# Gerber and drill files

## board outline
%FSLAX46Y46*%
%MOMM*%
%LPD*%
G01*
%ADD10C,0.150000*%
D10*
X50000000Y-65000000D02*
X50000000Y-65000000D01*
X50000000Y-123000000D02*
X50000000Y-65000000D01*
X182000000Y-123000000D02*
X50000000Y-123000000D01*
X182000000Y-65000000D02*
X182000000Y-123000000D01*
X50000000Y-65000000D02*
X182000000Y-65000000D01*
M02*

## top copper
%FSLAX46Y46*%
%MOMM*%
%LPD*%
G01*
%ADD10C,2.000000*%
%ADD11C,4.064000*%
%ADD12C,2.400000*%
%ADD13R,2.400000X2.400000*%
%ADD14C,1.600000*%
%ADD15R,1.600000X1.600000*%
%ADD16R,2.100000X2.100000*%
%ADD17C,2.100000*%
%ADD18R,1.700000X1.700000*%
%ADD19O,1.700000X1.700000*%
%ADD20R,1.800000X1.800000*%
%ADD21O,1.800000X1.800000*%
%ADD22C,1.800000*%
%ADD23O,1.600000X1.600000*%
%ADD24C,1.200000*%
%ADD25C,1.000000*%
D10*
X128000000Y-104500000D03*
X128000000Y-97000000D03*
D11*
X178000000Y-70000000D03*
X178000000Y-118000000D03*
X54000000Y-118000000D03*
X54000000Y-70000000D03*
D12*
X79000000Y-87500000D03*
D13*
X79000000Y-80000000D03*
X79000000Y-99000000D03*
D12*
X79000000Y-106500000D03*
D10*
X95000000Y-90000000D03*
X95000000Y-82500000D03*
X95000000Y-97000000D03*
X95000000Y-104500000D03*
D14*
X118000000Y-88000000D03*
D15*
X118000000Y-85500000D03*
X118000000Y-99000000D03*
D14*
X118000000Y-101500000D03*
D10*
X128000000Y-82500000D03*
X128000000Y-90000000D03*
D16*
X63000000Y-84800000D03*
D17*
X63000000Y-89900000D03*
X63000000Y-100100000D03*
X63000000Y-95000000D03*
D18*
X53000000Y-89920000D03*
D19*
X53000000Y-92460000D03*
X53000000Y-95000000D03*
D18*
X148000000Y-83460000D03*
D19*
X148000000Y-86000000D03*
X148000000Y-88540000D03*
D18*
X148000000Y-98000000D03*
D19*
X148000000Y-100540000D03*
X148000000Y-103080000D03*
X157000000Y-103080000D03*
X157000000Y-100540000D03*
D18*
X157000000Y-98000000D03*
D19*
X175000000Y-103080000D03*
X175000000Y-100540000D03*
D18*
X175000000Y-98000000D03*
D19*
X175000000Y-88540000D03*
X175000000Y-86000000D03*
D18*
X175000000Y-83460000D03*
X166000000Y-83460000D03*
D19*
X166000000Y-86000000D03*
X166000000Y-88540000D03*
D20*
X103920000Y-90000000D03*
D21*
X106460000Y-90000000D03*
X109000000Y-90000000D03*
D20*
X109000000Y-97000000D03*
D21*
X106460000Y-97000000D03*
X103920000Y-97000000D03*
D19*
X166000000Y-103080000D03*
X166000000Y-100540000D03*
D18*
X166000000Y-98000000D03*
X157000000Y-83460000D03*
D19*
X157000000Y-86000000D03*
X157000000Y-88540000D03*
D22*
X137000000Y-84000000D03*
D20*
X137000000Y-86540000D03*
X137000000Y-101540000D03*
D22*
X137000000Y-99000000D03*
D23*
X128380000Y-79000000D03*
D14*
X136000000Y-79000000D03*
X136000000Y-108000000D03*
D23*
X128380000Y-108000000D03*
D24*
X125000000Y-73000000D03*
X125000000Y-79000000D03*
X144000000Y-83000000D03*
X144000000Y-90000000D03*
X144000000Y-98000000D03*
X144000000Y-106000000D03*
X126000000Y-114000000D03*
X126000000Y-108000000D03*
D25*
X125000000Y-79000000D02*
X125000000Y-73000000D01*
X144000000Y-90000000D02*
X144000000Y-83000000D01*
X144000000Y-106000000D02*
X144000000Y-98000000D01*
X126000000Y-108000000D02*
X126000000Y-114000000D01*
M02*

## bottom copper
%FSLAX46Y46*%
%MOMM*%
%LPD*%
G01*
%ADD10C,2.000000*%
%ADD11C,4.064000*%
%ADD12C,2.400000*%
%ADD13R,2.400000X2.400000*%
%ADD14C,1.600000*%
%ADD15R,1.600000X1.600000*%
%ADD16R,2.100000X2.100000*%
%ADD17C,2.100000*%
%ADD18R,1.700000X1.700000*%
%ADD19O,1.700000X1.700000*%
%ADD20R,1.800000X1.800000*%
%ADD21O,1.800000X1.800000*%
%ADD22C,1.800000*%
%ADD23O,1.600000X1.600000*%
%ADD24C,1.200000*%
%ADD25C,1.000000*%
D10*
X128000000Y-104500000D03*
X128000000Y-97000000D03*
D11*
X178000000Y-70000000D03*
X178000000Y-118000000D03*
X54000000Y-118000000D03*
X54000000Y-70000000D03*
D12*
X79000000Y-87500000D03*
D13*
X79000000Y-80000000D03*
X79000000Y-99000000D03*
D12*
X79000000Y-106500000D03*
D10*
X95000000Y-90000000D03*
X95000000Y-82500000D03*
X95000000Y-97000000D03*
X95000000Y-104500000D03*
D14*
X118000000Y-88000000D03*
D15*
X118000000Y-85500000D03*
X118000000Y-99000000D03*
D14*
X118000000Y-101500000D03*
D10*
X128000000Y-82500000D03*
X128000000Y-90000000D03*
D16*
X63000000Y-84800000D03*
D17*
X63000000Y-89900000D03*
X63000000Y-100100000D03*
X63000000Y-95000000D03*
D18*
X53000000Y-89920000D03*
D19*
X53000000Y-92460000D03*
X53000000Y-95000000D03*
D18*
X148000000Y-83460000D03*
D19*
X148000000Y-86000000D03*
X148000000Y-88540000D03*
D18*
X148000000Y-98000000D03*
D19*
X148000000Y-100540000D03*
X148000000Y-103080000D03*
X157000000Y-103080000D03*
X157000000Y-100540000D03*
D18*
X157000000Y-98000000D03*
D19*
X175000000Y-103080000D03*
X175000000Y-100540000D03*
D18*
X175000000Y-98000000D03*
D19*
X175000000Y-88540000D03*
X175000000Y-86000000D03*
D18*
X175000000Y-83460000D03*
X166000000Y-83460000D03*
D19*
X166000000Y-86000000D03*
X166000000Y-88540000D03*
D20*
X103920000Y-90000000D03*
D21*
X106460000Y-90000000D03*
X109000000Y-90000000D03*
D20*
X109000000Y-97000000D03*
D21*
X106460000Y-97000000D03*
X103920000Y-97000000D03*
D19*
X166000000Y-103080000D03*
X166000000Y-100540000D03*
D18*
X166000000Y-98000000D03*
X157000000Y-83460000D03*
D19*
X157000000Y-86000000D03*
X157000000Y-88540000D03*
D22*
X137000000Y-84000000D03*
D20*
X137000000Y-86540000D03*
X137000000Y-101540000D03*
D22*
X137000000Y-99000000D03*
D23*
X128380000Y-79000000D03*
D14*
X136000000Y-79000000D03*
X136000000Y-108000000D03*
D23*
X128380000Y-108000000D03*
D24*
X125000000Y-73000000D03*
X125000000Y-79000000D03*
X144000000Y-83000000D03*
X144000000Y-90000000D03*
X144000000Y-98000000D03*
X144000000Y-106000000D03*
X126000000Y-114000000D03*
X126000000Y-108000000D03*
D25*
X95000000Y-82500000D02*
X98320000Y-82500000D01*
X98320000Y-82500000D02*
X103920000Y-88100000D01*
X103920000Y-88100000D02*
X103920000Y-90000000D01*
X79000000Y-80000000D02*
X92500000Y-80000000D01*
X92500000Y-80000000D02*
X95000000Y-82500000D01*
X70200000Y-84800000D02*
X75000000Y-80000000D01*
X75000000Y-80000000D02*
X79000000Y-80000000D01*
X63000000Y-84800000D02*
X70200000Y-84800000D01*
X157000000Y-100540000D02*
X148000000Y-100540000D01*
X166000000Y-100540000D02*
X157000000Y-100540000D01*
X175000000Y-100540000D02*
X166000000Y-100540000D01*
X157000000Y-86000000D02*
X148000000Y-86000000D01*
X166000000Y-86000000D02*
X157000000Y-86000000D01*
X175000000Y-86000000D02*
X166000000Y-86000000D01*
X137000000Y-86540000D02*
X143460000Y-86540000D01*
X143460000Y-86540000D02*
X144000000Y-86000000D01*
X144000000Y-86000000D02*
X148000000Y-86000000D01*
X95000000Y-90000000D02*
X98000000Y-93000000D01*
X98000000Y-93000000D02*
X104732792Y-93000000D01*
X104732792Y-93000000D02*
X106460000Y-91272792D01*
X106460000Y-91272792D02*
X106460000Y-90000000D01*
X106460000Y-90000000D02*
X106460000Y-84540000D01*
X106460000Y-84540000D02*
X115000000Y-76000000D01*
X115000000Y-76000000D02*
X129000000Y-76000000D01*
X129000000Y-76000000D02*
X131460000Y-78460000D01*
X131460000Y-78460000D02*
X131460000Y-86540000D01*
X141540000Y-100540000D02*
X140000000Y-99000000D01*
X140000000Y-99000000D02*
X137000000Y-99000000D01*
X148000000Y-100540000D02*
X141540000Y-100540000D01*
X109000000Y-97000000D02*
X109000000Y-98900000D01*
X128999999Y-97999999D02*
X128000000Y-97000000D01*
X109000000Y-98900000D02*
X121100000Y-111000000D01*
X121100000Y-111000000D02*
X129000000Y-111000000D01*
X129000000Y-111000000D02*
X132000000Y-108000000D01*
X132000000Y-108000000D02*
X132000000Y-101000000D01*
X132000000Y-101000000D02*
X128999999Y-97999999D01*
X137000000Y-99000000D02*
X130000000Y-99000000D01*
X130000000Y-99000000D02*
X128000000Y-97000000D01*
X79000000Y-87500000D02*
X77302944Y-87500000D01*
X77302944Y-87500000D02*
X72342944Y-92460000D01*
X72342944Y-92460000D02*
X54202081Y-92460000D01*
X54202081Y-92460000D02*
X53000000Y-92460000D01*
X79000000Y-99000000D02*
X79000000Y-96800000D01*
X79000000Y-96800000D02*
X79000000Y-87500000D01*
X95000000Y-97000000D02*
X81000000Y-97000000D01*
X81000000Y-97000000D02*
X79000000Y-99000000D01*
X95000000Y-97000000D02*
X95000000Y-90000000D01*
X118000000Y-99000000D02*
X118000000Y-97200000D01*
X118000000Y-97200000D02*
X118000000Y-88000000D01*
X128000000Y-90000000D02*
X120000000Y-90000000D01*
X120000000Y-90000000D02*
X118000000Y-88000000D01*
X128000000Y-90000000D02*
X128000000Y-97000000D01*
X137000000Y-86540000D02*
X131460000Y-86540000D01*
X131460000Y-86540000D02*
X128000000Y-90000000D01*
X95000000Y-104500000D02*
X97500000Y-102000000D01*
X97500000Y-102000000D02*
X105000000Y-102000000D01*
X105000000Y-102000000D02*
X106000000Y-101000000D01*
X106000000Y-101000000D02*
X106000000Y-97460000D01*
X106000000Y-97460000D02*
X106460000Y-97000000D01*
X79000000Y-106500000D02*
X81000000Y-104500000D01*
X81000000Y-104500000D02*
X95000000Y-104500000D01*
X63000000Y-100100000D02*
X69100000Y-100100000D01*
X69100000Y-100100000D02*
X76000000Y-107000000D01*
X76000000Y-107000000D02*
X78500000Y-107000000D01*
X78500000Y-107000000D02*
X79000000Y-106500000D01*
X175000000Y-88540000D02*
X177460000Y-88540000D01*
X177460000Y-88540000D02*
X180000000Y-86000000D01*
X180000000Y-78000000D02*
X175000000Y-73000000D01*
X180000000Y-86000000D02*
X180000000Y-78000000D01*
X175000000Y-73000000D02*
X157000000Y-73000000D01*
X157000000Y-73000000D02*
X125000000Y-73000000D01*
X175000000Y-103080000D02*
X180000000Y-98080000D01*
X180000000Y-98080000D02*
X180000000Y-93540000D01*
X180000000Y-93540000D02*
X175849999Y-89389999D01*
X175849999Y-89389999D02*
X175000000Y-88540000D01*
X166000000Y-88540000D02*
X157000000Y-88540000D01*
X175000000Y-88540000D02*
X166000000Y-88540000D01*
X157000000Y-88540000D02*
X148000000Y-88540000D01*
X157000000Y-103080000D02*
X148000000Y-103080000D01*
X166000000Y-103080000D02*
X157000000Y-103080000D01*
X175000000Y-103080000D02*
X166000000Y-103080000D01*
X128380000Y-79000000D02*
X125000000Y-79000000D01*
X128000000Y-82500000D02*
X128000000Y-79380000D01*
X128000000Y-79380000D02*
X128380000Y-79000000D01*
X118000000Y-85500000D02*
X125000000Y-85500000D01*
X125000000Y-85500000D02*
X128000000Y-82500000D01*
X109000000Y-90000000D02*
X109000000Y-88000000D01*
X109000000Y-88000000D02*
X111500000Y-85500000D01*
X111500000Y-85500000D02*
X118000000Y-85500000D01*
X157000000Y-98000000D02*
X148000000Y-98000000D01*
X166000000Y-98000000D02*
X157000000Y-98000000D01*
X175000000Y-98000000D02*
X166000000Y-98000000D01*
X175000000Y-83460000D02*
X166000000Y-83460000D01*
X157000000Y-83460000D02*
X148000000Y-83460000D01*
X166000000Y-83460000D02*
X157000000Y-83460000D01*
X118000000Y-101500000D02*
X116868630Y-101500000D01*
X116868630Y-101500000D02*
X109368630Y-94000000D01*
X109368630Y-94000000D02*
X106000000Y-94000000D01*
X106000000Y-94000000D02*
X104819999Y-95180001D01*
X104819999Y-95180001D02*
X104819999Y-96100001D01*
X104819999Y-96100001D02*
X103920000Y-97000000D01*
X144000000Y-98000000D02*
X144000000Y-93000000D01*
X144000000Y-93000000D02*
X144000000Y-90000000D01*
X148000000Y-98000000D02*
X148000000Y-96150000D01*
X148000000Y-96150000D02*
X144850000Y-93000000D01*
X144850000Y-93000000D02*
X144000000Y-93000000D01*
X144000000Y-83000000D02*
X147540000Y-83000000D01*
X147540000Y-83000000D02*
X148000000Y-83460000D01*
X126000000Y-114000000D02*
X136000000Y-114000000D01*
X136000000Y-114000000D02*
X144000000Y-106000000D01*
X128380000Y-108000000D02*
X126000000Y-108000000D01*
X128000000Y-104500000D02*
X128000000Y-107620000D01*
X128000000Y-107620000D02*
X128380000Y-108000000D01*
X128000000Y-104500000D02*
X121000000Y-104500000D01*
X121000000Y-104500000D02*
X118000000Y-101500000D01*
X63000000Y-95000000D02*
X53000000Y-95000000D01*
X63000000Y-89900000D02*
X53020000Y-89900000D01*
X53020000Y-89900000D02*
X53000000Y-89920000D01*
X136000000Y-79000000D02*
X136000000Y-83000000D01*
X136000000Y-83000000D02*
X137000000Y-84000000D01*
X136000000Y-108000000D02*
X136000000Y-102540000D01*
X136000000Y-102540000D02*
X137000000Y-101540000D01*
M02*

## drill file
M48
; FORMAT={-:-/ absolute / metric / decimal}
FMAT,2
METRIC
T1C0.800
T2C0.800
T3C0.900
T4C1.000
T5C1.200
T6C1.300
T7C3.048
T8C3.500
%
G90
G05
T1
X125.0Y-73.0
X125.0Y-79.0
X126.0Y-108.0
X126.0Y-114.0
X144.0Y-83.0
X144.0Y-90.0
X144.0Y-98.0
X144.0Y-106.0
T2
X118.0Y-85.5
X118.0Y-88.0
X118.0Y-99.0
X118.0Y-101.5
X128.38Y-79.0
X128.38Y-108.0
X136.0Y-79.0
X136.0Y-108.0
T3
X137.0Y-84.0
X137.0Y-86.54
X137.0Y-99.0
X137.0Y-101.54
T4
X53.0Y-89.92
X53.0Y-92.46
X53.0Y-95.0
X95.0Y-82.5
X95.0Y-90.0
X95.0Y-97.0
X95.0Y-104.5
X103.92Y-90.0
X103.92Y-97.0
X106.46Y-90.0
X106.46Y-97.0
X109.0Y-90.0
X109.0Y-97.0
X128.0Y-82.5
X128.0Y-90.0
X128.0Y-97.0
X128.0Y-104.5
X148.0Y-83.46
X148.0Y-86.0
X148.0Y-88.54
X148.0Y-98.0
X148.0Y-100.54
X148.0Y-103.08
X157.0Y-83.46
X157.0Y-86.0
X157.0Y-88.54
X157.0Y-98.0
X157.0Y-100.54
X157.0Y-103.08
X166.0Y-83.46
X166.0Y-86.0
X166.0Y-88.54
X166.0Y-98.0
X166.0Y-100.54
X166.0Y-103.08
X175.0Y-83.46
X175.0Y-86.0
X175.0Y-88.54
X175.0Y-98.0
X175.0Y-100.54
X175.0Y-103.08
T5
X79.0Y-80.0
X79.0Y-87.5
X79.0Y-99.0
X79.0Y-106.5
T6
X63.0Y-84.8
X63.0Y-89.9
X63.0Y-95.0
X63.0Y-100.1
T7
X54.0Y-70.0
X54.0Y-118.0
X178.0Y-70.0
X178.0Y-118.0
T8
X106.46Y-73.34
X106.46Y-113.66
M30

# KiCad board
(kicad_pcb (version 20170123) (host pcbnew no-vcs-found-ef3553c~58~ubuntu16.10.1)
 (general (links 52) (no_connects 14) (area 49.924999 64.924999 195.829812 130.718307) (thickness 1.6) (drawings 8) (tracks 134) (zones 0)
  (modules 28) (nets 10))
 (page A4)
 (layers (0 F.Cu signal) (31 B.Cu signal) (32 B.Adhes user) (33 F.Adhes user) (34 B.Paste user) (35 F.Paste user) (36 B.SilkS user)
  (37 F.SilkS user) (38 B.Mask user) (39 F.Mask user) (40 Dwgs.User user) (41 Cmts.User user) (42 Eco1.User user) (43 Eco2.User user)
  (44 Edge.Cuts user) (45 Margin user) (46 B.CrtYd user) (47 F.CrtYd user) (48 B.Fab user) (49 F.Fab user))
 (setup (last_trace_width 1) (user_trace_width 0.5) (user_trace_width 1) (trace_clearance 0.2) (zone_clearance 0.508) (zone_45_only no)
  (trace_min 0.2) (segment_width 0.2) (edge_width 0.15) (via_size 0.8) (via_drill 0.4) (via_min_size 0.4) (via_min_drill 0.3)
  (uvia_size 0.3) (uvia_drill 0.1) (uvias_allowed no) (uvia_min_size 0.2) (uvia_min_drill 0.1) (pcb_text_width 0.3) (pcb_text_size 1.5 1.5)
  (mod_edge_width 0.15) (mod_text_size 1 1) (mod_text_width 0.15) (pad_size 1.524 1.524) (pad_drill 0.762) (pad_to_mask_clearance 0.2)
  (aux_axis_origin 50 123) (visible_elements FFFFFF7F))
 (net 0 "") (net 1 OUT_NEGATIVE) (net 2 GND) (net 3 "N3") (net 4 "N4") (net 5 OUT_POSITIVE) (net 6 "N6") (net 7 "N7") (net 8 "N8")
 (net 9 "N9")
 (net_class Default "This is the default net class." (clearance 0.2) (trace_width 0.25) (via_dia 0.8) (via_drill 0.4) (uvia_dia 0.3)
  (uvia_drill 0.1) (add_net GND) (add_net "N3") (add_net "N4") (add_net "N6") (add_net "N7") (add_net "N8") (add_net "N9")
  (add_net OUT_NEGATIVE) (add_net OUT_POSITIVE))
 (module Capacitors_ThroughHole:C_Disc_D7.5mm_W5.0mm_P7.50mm (layer F.Cu) (at 128 97 270)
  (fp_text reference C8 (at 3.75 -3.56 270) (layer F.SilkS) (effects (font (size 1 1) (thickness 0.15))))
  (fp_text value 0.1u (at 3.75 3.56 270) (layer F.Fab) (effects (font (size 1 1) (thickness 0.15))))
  (pad 2 thru_hole circle (at 7.5 0 270) (size 2 2) (drill 1) (layers *.Cu *.Mask) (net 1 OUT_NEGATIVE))
  (pad 1 thru_hole circle (at 0 0 270) (size 2 2) (drill 1) (layers *.Cu *.Mask) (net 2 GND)))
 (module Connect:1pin (layer F.Cu) (at 178 70)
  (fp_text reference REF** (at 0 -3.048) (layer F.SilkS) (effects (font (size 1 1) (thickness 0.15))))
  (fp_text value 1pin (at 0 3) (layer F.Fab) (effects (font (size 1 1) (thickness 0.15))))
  (pad 1 thru_hole circle (at 0 0) (size 4.064 4.064) (drill 3.048) (layers *.Cu *.Mask)))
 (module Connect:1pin (layer F.Cu) (at 178 118)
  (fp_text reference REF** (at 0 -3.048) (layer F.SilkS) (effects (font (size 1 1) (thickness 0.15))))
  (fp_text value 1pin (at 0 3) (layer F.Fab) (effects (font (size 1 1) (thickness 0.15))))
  (pad 1 thru_hole circle (at 0 0) (size 4.064 4.064) (drill 3.048) (layers *.Cu *.Mask)))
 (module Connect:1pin (layer F.Cu) (at 54 118)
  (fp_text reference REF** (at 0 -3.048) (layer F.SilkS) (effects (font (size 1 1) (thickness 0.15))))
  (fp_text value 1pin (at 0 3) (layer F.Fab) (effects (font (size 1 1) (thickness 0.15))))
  (pad 1 thru_hole circle (at 0 0) (size 4.064 4.064) (drill 3.048) (layers *.Cu *.Mask)))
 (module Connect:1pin (layer F.Cu) (at 54 70)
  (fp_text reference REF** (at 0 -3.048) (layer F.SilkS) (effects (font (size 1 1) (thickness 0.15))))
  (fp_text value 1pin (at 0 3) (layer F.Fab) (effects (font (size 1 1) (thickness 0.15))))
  (pad 1 thru_hole circle (at 0 0) (size 4.064 4.064) (drill 3.048) (layers *.Cu *.Mask)))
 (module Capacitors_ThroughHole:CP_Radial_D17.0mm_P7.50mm (layer F.Cu) (at 79 80 270)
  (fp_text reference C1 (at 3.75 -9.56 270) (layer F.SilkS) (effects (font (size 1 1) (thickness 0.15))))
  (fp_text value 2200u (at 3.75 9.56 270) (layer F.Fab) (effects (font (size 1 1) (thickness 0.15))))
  (pad 2 thru_hole circle (at 7.5 0 270) (size 2.4 2.4) (drill 1.2) (layers *.Cu *.Mask) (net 2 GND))
  (pad 1 thru_hole rect (at 0 0 270) (size 2.4 2.4) (drill 1.2) (layers *.Cu *.Mask) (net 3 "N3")))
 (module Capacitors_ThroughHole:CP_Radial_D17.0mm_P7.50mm (layer F.Cu) (at 79 99 270)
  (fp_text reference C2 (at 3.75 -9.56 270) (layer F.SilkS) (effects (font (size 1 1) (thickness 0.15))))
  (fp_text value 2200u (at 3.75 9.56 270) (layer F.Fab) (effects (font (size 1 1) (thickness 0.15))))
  (pad 1 thru_hole rect (at 0 0 270) (size 2.4 2.4) (drill 1.2) (layers *.Cu *.Mask) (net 2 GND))
  (pad 2 thru_hole circle (at 7.5 0 270) (size 2.4 2.4) (drill 1.2) (layers *.Cu *.Mask) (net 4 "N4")))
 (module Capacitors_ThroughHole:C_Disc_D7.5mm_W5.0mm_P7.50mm (layer F.Cu) (at 95 82.5 270)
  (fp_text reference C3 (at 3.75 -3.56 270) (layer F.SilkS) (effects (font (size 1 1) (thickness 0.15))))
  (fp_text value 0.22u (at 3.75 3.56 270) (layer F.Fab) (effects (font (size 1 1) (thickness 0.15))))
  (pad 2 thru_hole circle (at 7.5 0 270) (size 2 2) (drill 1) (layers *.Cu *.Mask) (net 2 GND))
  (pad 1 thru_hole circle (at 0 0 270) (size 2 2) (drill 1) (layers *.Cu *.Mask) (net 3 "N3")))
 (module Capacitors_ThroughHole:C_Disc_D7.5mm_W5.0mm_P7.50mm (layer F.Cu) (at 95 97 270)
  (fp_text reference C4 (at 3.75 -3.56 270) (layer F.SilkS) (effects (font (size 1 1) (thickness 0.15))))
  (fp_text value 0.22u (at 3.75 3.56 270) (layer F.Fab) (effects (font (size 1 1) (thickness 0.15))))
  (pad 1 thru_hole circle (at 0 0 270) (size 2 2) (drill 1) (layers *.Cu *.Mask) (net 2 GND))
  (pad 2 thru_hole circle (at 7.5 0 270) (size 2 2) (drill 1) (layers *.Cu *.Mask) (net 4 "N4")))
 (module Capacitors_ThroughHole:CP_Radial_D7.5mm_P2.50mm (layer F.Cu) (at 118 85.5 270)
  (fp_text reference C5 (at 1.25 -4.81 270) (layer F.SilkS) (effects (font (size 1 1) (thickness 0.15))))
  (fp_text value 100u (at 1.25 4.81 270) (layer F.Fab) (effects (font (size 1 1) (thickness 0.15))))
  (pad 2 thru_hole circle (at 2.5 0 270) (size 1.6 1.6) (drill 0.8) (layers *.Cu *.Mask) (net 2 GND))
  (pad 1 thru_hole rect (at 0 0 270) (size 1.6 1.6) (drill 0.8) (layers *.Cu *.Mask) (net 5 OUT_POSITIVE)))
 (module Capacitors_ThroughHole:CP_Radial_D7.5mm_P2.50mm (layer F.Cu) (at 118 99 270)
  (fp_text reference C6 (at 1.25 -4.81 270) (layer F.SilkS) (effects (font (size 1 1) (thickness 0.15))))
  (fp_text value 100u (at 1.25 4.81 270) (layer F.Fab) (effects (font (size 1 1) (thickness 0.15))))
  (pad 1 thru_hole rect (at 0 0 270) (size 1.6 1.6) (drill 0.8) (layers *.Cu *.Mask) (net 2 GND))
  (pad 2 thru_hole circle (at 2.5 0 270) (size 1.6 1.6) (drill 0.8) (layers *.Cu *.Mask) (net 1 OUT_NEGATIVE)))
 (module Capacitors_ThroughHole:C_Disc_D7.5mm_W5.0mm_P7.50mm (layer F.Cu) (at 128 82.5 270)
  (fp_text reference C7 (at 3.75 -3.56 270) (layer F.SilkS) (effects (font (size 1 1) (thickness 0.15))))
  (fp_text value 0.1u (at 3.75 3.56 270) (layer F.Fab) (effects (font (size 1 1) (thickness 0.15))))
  (pad 1 thru_hole circle (at 0 0 270) (size 2 2) (drill 1) (layers *.Cu *.Mask) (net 5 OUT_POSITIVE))
  (pad 2 thru_hole circle (at 7.5 0 270) (size 2 2) (drill 1) (layers *.Cu *.Mask) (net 2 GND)))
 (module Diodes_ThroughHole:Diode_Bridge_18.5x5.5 (layer F.Cu) (at 63 84.8 270)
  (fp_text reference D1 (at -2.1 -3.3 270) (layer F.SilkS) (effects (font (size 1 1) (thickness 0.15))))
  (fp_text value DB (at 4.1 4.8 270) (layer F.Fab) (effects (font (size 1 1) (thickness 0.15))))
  (pad 3 thru_hole rect (at 0 0 270) (size 2.1 2.1) (drill 1.3) (layers *.Cu *.Mask) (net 3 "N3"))
  (pad 2 thru_hole circle (at 5.1 0 270) (size 2.1 2.1) (drill 1.3) (layers *.Cu *.Mask) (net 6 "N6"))
  (pad 1 thru_hole circle (at 15.3 0 270) (size 2.1 2.1) (drill 1.3) (layers *.Cu *.Mask) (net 4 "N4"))
  (pad 4 thru_hole circle (at 10.2 0 270) (size 2.1 2.1) (drill 1.3) (layers *.Cu *.Mask) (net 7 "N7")))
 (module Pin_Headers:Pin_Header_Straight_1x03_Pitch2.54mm (layer F.Cu) (at 53 89.92)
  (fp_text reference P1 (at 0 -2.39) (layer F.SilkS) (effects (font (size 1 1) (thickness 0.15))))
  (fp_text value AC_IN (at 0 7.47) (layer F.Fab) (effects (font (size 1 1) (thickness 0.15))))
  (pad 1 thru_hole rect (at 0 0) (size 1.7 1.7) (drill 1) (layers *.Cu *.Mask) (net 6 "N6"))
  (pad 2 thru_hole oval (at 0 2.54) (size 1.7 1.7) (drill 1) (layers *.Cu *.Mask) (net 2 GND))
  (pad 3 thru_hole oval (at 0 5.08) (size 1.7 1.7) (drill 1) (layers *.Cu *.Mask) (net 7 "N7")))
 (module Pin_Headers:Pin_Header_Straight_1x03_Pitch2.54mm (layer F.Cu) (at 148 83.46)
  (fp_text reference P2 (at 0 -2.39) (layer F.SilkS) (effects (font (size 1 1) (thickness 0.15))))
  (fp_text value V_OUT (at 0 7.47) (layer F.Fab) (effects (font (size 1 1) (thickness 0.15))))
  (pad 1 thru_hole rect (at 0 0) (size 1.7 1.7) (drill 1) (layers *.Cu *.Mask) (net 1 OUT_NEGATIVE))
  (pad 2 thru_hole oval (at 0 2.54) (size 1.7 1.7) (drill 1) (layers *.Cu *.Mask) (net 2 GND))
  (pad 3 thru_hole oval (at 0 5.08) (size 1.7 1.7) (drill 1) (layers *.Cu *.Mask) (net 5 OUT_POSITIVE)))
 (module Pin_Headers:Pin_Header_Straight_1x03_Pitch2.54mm (layer F.Cu) (at 148 98)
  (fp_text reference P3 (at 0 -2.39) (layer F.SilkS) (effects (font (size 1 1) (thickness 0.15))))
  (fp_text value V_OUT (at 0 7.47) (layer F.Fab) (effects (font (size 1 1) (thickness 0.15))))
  (pad 1 thru_hole rect (at 0 0) (size 1.7 1.7) (drill 1) (layers *.Cu *.Mask) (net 1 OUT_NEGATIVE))
  (pad 2 thru_hole oval (at 0 2.54) (size 1.7 1.7) (drill 1) (layers *.Cu *.Mask) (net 2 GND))
  (pad 3 thru_hole oval (at 0 5.08) (size 1.7 1.7) (drill 1) (layers *.Cu *.Mask) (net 5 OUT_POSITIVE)))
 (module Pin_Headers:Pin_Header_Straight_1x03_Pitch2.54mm (layer F.Cu) (at 157 98)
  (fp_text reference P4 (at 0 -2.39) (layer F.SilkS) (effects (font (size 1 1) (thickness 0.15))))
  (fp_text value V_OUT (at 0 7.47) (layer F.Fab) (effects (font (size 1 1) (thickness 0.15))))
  (pad 3 thru_hole oval (at 0 5.08) (size 1.7 1.7) (drill 1) (layers *.Cu *.Mask) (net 5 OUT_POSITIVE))
  (pad 2 thru_hole oval (at 0 2.54) (size 1.7 1.7) (drill 1) (layers *.Cu *.Mask) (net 2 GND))
  (pad 1 thru_hole rect (at 0 0) (size 1.7 1.7) (drill 1) (layers *.Cu *.Mask) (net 1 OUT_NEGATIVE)))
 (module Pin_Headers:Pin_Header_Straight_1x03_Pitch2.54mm (layer F.Cu) (at 175 98)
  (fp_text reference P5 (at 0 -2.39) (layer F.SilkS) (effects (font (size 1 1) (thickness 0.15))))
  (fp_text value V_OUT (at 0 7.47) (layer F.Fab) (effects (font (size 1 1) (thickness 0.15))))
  (pad 3 thru_hole oval (at 0 5.08) (size 1.7 1.7) (drill 1) (layers *.Cu *.Mask) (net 5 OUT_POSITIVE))
  (pad 2 thru_hole oval (at 0 2.54) (size 1.7 1.7) (drill 1) (layers *.Cu *.Mask) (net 2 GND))
  (pad 1 thru_hole rect (at 0 0) (size 1.7 1.7) (drill 1) (layers *.Cu *.Mask) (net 1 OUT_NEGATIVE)))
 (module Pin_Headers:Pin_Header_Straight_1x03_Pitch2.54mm (layer F.Cu) (at 175 83.46)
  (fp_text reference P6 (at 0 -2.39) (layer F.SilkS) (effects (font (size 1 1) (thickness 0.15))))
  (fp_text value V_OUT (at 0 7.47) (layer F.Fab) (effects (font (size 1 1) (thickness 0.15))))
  (pad 3 thru_hole oval (at 0 5.08) (size 1.7 1.7) (drill 1) (layers *.Cu *.Mask) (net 5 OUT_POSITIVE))
  (pad 2 thru_hole oval (at 0 2.54) (size 1.7 1.7) (drill 1) (layers *.Cu *.Mask) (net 2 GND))
  (pad 1 thru_hole rect (at 0 0) (size 1.7 1.7) (drill 1) (layers *.Cu *.Mask) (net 1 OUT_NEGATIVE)))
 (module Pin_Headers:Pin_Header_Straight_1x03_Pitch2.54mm (layer F.Cu) (at 166 83.46)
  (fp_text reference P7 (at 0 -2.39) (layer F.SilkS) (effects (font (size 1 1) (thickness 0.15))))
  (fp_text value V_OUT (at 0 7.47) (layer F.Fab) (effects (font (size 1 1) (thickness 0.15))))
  (pad 1 thru_hole rect (at 0 0) (size 1.7 1.7) (drill 1) (layers *.Cu *.Mask) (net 1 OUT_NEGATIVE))
  (pad 2 thru_hole oval (at 0 2.54) (size 1.7 1.7) (drill 1) (layers *.Cu *.Mask) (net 2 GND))
  (pad 3 thru_hole oval (at 0 5.08) (size 1.7 1.7) (drill 1) (layers *.Cu *.Mask) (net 5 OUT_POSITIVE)))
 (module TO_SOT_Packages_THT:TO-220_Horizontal (layer F.Cu) (at 103.92 90)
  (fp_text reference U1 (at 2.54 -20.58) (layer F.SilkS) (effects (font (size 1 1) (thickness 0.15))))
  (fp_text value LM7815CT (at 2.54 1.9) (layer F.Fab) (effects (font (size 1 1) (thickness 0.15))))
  (pad None np_thru_hole oval (at 2.54 -16.66) (size 3.5 3.5) (drill 3.5) (layers *.Cu *.Mask))
  (pad 1 thru_hole rect (at 0 0) (size 1.8 1.8) (drill 1) (layers *.Cu *.Mask) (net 3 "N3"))
  (pad 2 thru_hole oval (at 2.54 0) (size 1.8 1.8) (drill 1) (layers *.Cu *.Mask) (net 2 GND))
  (pad 3 thru_hole oval (at 5.08 0) (size 1.8 1.8) (drill 1) (layers *.Cu *.Mask) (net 5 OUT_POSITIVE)))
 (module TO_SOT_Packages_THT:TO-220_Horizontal (layer F.Cu) (at 109 97 180)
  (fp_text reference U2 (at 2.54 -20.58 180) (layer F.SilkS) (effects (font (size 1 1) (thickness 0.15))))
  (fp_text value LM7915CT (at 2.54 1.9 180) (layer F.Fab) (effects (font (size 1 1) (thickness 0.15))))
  (pad None np_thru_hole oval (at 2.54 -16.66 180) (size 3.5 3.5) (drill 3.5) (layers *.Cu *.Mask))
  (pad 1 thru_hole rect (at 0 0 180) (size 1.8 1.8) (drill 1) (layers *.Cu *.Mask) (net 2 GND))
  (pad 2 thru_hole oval (at 2.54 0 180) (size 1.8 1.8) (drill 1) (layers *.Cu *.Mask) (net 4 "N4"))
  (pad 3 thru_hole oval (at 5.08 0 180) (size 1.8 1.8) (drill 1) (layers *.Cu *.Mask) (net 1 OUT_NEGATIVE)))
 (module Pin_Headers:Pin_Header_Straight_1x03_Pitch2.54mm (layer F.Cu) (at 166 98)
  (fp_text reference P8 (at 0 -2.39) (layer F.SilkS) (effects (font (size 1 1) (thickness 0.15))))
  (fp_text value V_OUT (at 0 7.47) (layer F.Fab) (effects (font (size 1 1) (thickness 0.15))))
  (pad 3 thru_hole oval (at 0 5.08) (size 1.7 1.7) (drill 1) (layers *.Cu *.Mask) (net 5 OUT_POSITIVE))
  (pad 2 thru_hole oval (at 0 2.54) (size 1.7 1.7) (drill 1) (layers *.Cu *.Mask) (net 2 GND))
  (pad 1 thru_hole rect (at 0 0) (size 1.7 1.7) (drill 1) (layers *.Cu *.Mask) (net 1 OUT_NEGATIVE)))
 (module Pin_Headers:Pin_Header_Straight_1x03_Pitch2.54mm (layer F.Cu) (at 157 83.46)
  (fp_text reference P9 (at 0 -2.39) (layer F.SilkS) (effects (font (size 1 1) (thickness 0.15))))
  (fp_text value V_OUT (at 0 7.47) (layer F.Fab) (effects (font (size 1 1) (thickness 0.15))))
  (pad 1 thru_hole rect (at 0 0) (size 1.7 1.7) (drill 1) (layers *.Cu *.Mask) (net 1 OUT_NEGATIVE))
  (pad 2 thru_hole oval (at 0 2.54) (size 1.7 1.7) (drill 1) (layers *.Cu *.Mask) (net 2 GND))
  (pad 3 thru_hole oval (at 0 5.08) (size 1.7 1.7) (drill 1) (layers *.Cu *.Mask) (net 5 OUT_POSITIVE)))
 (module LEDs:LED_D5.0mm (layer F.Cu) (at 137 86.54 90)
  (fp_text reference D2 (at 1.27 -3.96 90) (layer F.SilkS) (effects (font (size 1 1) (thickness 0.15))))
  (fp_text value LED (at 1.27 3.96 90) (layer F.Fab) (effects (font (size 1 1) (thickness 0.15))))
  (pad 2 thru_hole circle (at 2.54 0 90) (size 1.8 1.8) (drill 0.9) (layers *.Cu *.Mask) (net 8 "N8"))
  (pad 1 thru_hole rect (at 0 0 90) (size 1.8 1.8) (drill 0.9) (layers *.Cu *.Mask) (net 2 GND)))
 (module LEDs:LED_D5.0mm (layer F.Cu) (at 137 101.54 90)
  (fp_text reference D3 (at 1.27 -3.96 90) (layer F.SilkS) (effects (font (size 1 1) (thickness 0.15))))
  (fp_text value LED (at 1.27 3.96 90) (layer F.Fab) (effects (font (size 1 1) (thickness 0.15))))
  (pad 1 thru_hole rect (at 0 0 90) (size 1.8 1.8) (drill 0.9) (layers *.Cu *.Mask) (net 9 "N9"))
  (pad 2 thru_hole circle (at 2.54 0 90) (size 1.8 1.8) (drill 0.9) (layers *.Cu *.Mask) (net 2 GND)))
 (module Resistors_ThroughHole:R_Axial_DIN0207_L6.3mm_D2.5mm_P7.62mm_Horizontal (layer F.Cu) (at 136 79 180)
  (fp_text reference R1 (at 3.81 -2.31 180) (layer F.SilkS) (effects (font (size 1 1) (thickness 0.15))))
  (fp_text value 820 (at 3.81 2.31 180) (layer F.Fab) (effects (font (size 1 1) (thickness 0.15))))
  (pad 2 thru_hole oval (at 7.62 0 180) (size 1.6 1.6) (drill 0.8) (layers *.Cu *.Mask) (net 5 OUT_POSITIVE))
  (pad 1 thru_hole circle (at 0 0 180) (size 1.6 1.6) (drill 0.8) (layers *.Cu *.Mask) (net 8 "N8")))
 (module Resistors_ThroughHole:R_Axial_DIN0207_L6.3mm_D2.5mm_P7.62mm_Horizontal (layer F.Cu) (at 136 108 180)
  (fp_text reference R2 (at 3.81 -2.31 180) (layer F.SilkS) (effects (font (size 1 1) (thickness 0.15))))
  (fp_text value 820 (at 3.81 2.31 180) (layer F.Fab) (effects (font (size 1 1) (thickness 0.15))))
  (pad 1 thru_hole circle (at 0 0 180) (size 1.6 1.6) (drill 0.8) (layers *.Cu *.Mask) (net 9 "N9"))
  (pad 2 thru_hole oval (at 7.62 0 180) (size 1.6 1.6) (drill 0.8) (layers *.Cu *.Mask) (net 1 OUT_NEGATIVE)))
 (gr_line (start 50 65) (end 50 65) (layer Edge.Cuts) (width 0.15))
 (gr_line (start 50 123) (end 50 65) (layer Edge.Cuts) (width 0.15))
 (gr_line (start 182 123) (end 50 123) (layer Edge.Cuts) (width 0.15))
 (gr_line (start 182 65) (end 182 123) (layer Edge.Cuts) (width 0.15))
 (gr_line (start 50 65) (end 182 65) (layer Edge.Cuts) (width 0.15))
 (segment (start 95 82.5) (end 98.32 82.5) (width 1) (layer B.Cu) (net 3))
 (segment (start 98.32 82.5) (end 103.92 88.1) (width 1) (layer B.Cu) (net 3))
 (segment (start 103.92 88.1) (end 103.92 90) (width 1) (layer B.Cu) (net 3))
 (segment (start 79 80) (end 92.5 80) (width 1) (layer B.Cu) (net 3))
 (segment (start 92.5 80) (end 95 82.5) (width 1) (layer B.Cu) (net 3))
 (segment (start 70.2 84.8) (end 75 80) (width 1) (layer B.Cu) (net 3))
 (segment (start 75 80) (end 79 80) (width 1) (layer B.Cu) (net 3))
 (segment (start 63 84.8) (end 70.2 84.8) (width 1) (layer B.Cu) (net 3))
 (segment (start 157 100.54) (end 148 100.54) (width 1) (layer B.Cu) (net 2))
 (segment (start 166 100.54) (end 157 100.54) (width 1) (layer B.Cu) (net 2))
 (segment (start 175 100.54) (end 166 100.54) (width 1) (layer B.Cu) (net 2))
 (segment (start 157 86) (end 148 86) (width 1) (layer B.Cu) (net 2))
 (segment (start 166 86) (end 157 86) (width 1) (layer B.Cu) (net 2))
 (segment (start 175 86) (end 166 86) (width 1) (layer B.Cu) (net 2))
 (segment (start 137 86.54) (end 143.46 86.54) (width 1) (layer B.Cu) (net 2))
 (segment (start 143.46 86.54) (end 144 86) (width 1) (layer B.Cu) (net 2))
 (segment (start 144 86) (end 148 86) (width 1) (layer B.Cu) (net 2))
 (segment (start 95 90) (end 98 93) (width 1) (layer B.Cu) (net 2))
 (segment (start 98 93) (end 104.732792 93) (width 1) (layer B.Cu) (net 2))
 (segment (start 104.732792 93) (end 106.46 91.272792) (width 1) (layer B.Cu) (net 2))
 (segment (start 106.46 91.272792) (end 106.46 90) (width 1) (layer B.Cu) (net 2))
 (segment (start 106.46 90) (end 106.46 84.54) (width 1) (layer B.Cu) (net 2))
 (segment (start 106.46 84.54) (end 115 76) (width 1) (layer B.Cu) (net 2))
 (segment (start 115 76) (end 129 76) (width 1) (layer B.Cu) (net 2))
 (segment (start 129 76) (end 131.46 78.46) (width 1) (layer B.Cu) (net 2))
 (segment (start 131.46 78.46) (end 131.46 86.54) (width 1) (layer B.Cu) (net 2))
 (segment (start 141.54 100.54) (end 140 99) (width 1) (layer B.Cu) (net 2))
 (segment (start 140 99) (end 137 99) (width 1) (layer B.Cu) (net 2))
 (segment (start 148 100.54) (end 141.54 100.54) (width 1) (layer B.Cu) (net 2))
 (segment (start 109 97) (end 109 98.9) (width 1) (layer B.Cu) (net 2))
 (segment (start 128.999999 97.999999) (end 128 97) (width 1) (layer B.Cu) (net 2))
 (segment (start 109 98.9) (end 121.1 111) (width 1) (layer B.Cu) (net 2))
 (segment (start 121.1 111) (end 129 111) (width 1) (layer B.Cu) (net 2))
 (segment (start 129 111) (end 132 108) (width 1) (layer B.Cu) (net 2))
 (segment (start 132 108) (end 132 101) (width 1) (layer B.Cu) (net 2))
 (segment (start 132 101) (end 128.999999 97.999999) (width 1) (layer B.Cu) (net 2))
 (segment (start 137 99) (end 130 99) (width 1) (layer B.Cu) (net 2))
 (segment (start 130 99) (end 128 97) (width 1) (layer B.Cu) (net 2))
 (segment (start 79 87.5) (end 77.302944 87.5) (width 1) (layer B.Cu) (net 2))
 (segment (start 77.302944 87.5) (end 72.342944 92.46) (width 1) (layer B.Cu) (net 2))
 (segment (start 72.342944 92.46) (end 54.202081 92.46) (width 1) (layer B.Cu) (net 2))
 (segment (start 54.202081 92.46) (end 53 92.46) (width 1) (layer B.Cu) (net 2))
 (segment (start 79 99) (end 79 96.8) (width 1) (layer B.Cu) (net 2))
 (segment (start 79 96.8) (end 79 87.5) (width 1) (layer B.Cu) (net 2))
 (segment (start 95 97) (end 81 97) (width 1) (layer B.Cu) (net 2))
 (segment (start 81 97) (end 79 99) (width 1) (layer B.Cu) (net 2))
 (segment (start 95 97) (end 95 90) (width 1) (layer B.Cu) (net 2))
 (segment (start 118 99) (end 118 97.2) (width 1) (layer B.Cu) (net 2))
 (segment (start 118 97.2) (end 118 88) (width 1) (layer B.Cu) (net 2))
 (segment (start 128 90) (end 120 90) (width 1) (layer B.Cu) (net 2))
 (segment (start 120 90) (end 118 88) (width 1) (layer B.Cu) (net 2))
 (segment (start 128 90) (end 128 97) (width 1) (layer B.Cu) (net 2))
 (segment (start 137 86.54) (end 131.46 86.54) (width 1) (layer B.Cu) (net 2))
 (segment (start 131.46 86.54) (end 128 90) (width 1) (layer B.Cu) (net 2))
 (segment (start 95 104.5) (end 97.5 102) (width 1) (layer B.Cu) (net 4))
 (segment (start 97.5 102) (end 105 102) (width 1) (layer B.Cu) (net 4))
 (segment (start 105 102) (end 106 101) (width 1) (layer B.Cu) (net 4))
 (segment (start 106 101) (end 106 97.46) (width 1) (layer B.Cu) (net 4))
 (segment (start 106 97.46) (end 106.46 97) (width 1) (layer B.Cu) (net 4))
 (segment (start 79 106.5) (end 81 104.5) (width 1) (layer B.Cu) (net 4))
 (segment (start 81 104.5) (end 95 104.5) (width 1) (layer B.Cu) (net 4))
 (segment (start 63 100.1) (end 69.1 100.1) (width 1) (layer B.Cu) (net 4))
 (segment (start 69.1 100.1) (end 76 107) (width 1) (layer B.Cu) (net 4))
 (segment (start 76 107) (end 78.5 107) (width 1) (layer B.Cu) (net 4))
 (segment (start 78.5 107) (end 79 106.5) (width 1) (layer B.Cu) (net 4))
 (segment (start 175 88.54) (end 177.46 88.54) (width 1) (layer B.Cu) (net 5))
 (segment (start 177.46 88.54) (end 180 86) (width 1) (layer B.Cu) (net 5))
 (segment (start 180 78) (end 175 73) (width 1) (layer B.Cu) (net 5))
 (segment (start 180 86) (end 180 78) (width 1) (layer B.Cu) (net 5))
 (segment (start 175 73) (end 157 73) (width 1) (layer B.Cu) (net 5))
 (segment (start 157 73) (end 125 73) (width 1) (layer B.Cu) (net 5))
 (segment (start 175 103.08) (end 180 98.08) (width 1) (layer B.Cu) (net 5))
 (segment (start 180 98.08) (end 180 93.54) (width 1) (layer B.Cu) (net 5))
 (segment (start 180 93.54) (end 175.849999 89.389999) (width 1) (layer B.Cu) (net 5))
 (segment (start 175.849999 89.389999) (end 175 88.54) (width 1) (layer B.Cu) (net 5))
 (segment (start 166 88.54) (end 157 88.54) (width 1) (layer B.Cu) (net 5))
 (segment (start 175 88.54) (end 166 88.54) (width 1) (layer B.Cu) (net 5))
 (segment (start 157 88.54) (end 148 88.54) (width 1) (layer B.Cu) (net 5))
 (segment (start 157 103.08) (end 148 103.08) (width 1) (layer B.Cu) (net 5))
 (segment (start 166 103.08) (end 157 103.08) (width 1) (layer B.Cu) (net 5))
 (segment (start 175 103.08) (end 166 103.08) (width 1) (layer B.Cu) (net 5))
 (segment (start 125 79) (end 125 73) (width 1) (layer F.Cu) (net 5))
 (via (at 125 73) (size 1.2) (drill 0.8) (layers F.Cu B.Cu) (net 5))
 (via (at 125 79) (size 1.2) (drill 0.8) (layers F.Cu B.Cu) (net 5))
 (segment (start 128.38 79) (end 125 79) (width 1) (layer B.Cu) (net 5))
 (segment (start 128 82.5) (end 128 79.38) (width 1) (layer B.Cu) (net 5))
 (segment (start 128 79.38) (end 128.38 79) (width 1) (layer B.Cu) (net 5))
 (segment (start 118 85.5) (end 125 85.5) (width 1) (layer B.Cu) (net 5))
 (segment (start 125 85.5) (end 128 82.5) (width 1) (layer B.Cu) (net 5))
 (segment (start 109 90) (end 109 88) (width 1) (layer B.Cu) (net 5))
 (segment (start 109 88) (end 111.5 85.5) (width 1) (layer B.Cu) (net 5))
 (segment (start 111.5 85.5) (end 118 85.5) (width 1) (layer B.Cu) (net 5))
 (segment (start 157 98) (end 148 98) (width 1) (layer B.Cu) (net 1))
 (segment (start 166 98) (end 157 98) (width 1) (layer B.Cu) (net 1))
 (segment (start 175 98) (end 166 98) (width 1) (layer B.Cu) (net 1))
 (segment (start 175 83.46) (end 166 83.46) (width 1) (layer B.Cu) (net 1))
 (segment (start 157 83.46) (end 148 83.46) (width 1) (layer B.Cu) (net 1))
 (segment (start 166 83.46) (end 157 83.46) (width 1) (layer B.Cu) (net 1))
 (segment (start 118 101.5) (end 116.86863 101.5) (width 1) (layer B.Cu) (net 1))
 (segment (start 116.86863 101.5) (end 109.36863 94) (width 1) (layer B.Cu) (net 1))
 (segment (start 109.36863 94) (end 106 94) (width 1) (layer B.Cu) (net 1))
 (segment (start 106 94) (end 104.819999 95.180001) (width 1) (layer B.Cu) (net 1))
 (segment (start 104.819999 95.180001) (end 104.819999 96.100001) (width 1) (layer B.Cu) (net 1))
 (segment (start 104.819999 96.100001) (end 103.92 97) (width 1) (layer B.Cu) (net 1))
 (segment (start 144 98) (end 144 93) (width 1) (layer B.Cu) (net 1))
 (segment (start 144 93) (end 144 90) (width 1) (layer B.Cu) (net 1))
 (segment (start 148 98) (end 148 96.15) (width 1) (layer B.Cu) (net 1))
 (segment (start 148 96.15) (end 144.85 93) (width 1) (layer B.Cu) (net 1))
 (segment (start 144.85 93) (end 144 93) (width 1) (layer B.Cu) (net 1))
 (segment (start 144 83) (end 147.54 83) (width 1) (layer B.Cu) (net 1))
 (segment (start 147.54 83) (end 148 83.46) (width 1) (layer B.Cu) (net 1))
 (segment (start 144 90) (end 144 83) (width 1) (layer F.Cu) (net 1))
 (via (at 144 83) (size 1.2) (drill 0.8) (layers F.Cu B.Cu) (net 1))
 (via (at 144 90) (size 1.2) (drill 0.8) (layers F.Cu B.Cu) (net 1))
 (segment (start 144 106) (end 144 98) (width 1) (layer F.Cu) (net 1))
 (via (at 144 98) (size 1.2) (drill 0.8) (layers F.Cu B.Cu) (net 1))
 (segment (start 126 114) (end 136 114) (width 1) (layer B.Cu) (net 1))
 (via (at 144 106) (size 1.2) (drill 0.8) (layers F.Cu B.Cu) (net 1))
 (segment (start 136 114) (end 144 106) (width 1) (layer B.Cu) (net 1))
 (segment (start 126 108) (end 126 114) (width 1) (layer F.Cu) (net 1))
 (via (at 126 114) (size 1.2) (drill 0.8) (layers F.Cu B.Cu) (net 1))
 (segment (start 128.38 108) (end 126 108) (width 1) (layer B.Cu) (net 1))
 (via (at 126 108) (size 1.2) (drill 0.8) (layers F.Cu B.Cu) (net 1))
 (segment (start 128 104.5) (end 128 107.62) (width 1) (layer B.Cu) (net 1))
 (segment (start 128 107.62) (end 128.38 108) (width 1) (layer B.Cu) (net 1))
 (segment (start 128 104.5) (end 121 104.5) (width 1) (layer B.Cu) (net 1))
 (segment (start 121 104.5) (end 118 101.5) (width 1) (layer B.Cu) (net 1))
 (segment (start 63 95) (end 53 95) (width 1) (layer B.Cu) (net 7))
 (segment (start 63 89.9) (end 53.02 89.9) (width 1) (layer B.Cu) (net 6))
 (segment (start 53.02 89.9) (end 53 89.92) (width 1) (layer B.Cu) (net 6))
 (segment (start 136 79) (end 136 83) (width 1) (layer B.Cu) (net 8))
 (segment (start 136 83) (end 137 84) (width 1) (layer B.Cu) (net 8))
 (segment (start 136 108) (end 136 102.54) (width 1) (layer B.Cu) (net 9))
 (segment (start 136 102.54) (end 137 101.54) (width 1) (layer B.Cu) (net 9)))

